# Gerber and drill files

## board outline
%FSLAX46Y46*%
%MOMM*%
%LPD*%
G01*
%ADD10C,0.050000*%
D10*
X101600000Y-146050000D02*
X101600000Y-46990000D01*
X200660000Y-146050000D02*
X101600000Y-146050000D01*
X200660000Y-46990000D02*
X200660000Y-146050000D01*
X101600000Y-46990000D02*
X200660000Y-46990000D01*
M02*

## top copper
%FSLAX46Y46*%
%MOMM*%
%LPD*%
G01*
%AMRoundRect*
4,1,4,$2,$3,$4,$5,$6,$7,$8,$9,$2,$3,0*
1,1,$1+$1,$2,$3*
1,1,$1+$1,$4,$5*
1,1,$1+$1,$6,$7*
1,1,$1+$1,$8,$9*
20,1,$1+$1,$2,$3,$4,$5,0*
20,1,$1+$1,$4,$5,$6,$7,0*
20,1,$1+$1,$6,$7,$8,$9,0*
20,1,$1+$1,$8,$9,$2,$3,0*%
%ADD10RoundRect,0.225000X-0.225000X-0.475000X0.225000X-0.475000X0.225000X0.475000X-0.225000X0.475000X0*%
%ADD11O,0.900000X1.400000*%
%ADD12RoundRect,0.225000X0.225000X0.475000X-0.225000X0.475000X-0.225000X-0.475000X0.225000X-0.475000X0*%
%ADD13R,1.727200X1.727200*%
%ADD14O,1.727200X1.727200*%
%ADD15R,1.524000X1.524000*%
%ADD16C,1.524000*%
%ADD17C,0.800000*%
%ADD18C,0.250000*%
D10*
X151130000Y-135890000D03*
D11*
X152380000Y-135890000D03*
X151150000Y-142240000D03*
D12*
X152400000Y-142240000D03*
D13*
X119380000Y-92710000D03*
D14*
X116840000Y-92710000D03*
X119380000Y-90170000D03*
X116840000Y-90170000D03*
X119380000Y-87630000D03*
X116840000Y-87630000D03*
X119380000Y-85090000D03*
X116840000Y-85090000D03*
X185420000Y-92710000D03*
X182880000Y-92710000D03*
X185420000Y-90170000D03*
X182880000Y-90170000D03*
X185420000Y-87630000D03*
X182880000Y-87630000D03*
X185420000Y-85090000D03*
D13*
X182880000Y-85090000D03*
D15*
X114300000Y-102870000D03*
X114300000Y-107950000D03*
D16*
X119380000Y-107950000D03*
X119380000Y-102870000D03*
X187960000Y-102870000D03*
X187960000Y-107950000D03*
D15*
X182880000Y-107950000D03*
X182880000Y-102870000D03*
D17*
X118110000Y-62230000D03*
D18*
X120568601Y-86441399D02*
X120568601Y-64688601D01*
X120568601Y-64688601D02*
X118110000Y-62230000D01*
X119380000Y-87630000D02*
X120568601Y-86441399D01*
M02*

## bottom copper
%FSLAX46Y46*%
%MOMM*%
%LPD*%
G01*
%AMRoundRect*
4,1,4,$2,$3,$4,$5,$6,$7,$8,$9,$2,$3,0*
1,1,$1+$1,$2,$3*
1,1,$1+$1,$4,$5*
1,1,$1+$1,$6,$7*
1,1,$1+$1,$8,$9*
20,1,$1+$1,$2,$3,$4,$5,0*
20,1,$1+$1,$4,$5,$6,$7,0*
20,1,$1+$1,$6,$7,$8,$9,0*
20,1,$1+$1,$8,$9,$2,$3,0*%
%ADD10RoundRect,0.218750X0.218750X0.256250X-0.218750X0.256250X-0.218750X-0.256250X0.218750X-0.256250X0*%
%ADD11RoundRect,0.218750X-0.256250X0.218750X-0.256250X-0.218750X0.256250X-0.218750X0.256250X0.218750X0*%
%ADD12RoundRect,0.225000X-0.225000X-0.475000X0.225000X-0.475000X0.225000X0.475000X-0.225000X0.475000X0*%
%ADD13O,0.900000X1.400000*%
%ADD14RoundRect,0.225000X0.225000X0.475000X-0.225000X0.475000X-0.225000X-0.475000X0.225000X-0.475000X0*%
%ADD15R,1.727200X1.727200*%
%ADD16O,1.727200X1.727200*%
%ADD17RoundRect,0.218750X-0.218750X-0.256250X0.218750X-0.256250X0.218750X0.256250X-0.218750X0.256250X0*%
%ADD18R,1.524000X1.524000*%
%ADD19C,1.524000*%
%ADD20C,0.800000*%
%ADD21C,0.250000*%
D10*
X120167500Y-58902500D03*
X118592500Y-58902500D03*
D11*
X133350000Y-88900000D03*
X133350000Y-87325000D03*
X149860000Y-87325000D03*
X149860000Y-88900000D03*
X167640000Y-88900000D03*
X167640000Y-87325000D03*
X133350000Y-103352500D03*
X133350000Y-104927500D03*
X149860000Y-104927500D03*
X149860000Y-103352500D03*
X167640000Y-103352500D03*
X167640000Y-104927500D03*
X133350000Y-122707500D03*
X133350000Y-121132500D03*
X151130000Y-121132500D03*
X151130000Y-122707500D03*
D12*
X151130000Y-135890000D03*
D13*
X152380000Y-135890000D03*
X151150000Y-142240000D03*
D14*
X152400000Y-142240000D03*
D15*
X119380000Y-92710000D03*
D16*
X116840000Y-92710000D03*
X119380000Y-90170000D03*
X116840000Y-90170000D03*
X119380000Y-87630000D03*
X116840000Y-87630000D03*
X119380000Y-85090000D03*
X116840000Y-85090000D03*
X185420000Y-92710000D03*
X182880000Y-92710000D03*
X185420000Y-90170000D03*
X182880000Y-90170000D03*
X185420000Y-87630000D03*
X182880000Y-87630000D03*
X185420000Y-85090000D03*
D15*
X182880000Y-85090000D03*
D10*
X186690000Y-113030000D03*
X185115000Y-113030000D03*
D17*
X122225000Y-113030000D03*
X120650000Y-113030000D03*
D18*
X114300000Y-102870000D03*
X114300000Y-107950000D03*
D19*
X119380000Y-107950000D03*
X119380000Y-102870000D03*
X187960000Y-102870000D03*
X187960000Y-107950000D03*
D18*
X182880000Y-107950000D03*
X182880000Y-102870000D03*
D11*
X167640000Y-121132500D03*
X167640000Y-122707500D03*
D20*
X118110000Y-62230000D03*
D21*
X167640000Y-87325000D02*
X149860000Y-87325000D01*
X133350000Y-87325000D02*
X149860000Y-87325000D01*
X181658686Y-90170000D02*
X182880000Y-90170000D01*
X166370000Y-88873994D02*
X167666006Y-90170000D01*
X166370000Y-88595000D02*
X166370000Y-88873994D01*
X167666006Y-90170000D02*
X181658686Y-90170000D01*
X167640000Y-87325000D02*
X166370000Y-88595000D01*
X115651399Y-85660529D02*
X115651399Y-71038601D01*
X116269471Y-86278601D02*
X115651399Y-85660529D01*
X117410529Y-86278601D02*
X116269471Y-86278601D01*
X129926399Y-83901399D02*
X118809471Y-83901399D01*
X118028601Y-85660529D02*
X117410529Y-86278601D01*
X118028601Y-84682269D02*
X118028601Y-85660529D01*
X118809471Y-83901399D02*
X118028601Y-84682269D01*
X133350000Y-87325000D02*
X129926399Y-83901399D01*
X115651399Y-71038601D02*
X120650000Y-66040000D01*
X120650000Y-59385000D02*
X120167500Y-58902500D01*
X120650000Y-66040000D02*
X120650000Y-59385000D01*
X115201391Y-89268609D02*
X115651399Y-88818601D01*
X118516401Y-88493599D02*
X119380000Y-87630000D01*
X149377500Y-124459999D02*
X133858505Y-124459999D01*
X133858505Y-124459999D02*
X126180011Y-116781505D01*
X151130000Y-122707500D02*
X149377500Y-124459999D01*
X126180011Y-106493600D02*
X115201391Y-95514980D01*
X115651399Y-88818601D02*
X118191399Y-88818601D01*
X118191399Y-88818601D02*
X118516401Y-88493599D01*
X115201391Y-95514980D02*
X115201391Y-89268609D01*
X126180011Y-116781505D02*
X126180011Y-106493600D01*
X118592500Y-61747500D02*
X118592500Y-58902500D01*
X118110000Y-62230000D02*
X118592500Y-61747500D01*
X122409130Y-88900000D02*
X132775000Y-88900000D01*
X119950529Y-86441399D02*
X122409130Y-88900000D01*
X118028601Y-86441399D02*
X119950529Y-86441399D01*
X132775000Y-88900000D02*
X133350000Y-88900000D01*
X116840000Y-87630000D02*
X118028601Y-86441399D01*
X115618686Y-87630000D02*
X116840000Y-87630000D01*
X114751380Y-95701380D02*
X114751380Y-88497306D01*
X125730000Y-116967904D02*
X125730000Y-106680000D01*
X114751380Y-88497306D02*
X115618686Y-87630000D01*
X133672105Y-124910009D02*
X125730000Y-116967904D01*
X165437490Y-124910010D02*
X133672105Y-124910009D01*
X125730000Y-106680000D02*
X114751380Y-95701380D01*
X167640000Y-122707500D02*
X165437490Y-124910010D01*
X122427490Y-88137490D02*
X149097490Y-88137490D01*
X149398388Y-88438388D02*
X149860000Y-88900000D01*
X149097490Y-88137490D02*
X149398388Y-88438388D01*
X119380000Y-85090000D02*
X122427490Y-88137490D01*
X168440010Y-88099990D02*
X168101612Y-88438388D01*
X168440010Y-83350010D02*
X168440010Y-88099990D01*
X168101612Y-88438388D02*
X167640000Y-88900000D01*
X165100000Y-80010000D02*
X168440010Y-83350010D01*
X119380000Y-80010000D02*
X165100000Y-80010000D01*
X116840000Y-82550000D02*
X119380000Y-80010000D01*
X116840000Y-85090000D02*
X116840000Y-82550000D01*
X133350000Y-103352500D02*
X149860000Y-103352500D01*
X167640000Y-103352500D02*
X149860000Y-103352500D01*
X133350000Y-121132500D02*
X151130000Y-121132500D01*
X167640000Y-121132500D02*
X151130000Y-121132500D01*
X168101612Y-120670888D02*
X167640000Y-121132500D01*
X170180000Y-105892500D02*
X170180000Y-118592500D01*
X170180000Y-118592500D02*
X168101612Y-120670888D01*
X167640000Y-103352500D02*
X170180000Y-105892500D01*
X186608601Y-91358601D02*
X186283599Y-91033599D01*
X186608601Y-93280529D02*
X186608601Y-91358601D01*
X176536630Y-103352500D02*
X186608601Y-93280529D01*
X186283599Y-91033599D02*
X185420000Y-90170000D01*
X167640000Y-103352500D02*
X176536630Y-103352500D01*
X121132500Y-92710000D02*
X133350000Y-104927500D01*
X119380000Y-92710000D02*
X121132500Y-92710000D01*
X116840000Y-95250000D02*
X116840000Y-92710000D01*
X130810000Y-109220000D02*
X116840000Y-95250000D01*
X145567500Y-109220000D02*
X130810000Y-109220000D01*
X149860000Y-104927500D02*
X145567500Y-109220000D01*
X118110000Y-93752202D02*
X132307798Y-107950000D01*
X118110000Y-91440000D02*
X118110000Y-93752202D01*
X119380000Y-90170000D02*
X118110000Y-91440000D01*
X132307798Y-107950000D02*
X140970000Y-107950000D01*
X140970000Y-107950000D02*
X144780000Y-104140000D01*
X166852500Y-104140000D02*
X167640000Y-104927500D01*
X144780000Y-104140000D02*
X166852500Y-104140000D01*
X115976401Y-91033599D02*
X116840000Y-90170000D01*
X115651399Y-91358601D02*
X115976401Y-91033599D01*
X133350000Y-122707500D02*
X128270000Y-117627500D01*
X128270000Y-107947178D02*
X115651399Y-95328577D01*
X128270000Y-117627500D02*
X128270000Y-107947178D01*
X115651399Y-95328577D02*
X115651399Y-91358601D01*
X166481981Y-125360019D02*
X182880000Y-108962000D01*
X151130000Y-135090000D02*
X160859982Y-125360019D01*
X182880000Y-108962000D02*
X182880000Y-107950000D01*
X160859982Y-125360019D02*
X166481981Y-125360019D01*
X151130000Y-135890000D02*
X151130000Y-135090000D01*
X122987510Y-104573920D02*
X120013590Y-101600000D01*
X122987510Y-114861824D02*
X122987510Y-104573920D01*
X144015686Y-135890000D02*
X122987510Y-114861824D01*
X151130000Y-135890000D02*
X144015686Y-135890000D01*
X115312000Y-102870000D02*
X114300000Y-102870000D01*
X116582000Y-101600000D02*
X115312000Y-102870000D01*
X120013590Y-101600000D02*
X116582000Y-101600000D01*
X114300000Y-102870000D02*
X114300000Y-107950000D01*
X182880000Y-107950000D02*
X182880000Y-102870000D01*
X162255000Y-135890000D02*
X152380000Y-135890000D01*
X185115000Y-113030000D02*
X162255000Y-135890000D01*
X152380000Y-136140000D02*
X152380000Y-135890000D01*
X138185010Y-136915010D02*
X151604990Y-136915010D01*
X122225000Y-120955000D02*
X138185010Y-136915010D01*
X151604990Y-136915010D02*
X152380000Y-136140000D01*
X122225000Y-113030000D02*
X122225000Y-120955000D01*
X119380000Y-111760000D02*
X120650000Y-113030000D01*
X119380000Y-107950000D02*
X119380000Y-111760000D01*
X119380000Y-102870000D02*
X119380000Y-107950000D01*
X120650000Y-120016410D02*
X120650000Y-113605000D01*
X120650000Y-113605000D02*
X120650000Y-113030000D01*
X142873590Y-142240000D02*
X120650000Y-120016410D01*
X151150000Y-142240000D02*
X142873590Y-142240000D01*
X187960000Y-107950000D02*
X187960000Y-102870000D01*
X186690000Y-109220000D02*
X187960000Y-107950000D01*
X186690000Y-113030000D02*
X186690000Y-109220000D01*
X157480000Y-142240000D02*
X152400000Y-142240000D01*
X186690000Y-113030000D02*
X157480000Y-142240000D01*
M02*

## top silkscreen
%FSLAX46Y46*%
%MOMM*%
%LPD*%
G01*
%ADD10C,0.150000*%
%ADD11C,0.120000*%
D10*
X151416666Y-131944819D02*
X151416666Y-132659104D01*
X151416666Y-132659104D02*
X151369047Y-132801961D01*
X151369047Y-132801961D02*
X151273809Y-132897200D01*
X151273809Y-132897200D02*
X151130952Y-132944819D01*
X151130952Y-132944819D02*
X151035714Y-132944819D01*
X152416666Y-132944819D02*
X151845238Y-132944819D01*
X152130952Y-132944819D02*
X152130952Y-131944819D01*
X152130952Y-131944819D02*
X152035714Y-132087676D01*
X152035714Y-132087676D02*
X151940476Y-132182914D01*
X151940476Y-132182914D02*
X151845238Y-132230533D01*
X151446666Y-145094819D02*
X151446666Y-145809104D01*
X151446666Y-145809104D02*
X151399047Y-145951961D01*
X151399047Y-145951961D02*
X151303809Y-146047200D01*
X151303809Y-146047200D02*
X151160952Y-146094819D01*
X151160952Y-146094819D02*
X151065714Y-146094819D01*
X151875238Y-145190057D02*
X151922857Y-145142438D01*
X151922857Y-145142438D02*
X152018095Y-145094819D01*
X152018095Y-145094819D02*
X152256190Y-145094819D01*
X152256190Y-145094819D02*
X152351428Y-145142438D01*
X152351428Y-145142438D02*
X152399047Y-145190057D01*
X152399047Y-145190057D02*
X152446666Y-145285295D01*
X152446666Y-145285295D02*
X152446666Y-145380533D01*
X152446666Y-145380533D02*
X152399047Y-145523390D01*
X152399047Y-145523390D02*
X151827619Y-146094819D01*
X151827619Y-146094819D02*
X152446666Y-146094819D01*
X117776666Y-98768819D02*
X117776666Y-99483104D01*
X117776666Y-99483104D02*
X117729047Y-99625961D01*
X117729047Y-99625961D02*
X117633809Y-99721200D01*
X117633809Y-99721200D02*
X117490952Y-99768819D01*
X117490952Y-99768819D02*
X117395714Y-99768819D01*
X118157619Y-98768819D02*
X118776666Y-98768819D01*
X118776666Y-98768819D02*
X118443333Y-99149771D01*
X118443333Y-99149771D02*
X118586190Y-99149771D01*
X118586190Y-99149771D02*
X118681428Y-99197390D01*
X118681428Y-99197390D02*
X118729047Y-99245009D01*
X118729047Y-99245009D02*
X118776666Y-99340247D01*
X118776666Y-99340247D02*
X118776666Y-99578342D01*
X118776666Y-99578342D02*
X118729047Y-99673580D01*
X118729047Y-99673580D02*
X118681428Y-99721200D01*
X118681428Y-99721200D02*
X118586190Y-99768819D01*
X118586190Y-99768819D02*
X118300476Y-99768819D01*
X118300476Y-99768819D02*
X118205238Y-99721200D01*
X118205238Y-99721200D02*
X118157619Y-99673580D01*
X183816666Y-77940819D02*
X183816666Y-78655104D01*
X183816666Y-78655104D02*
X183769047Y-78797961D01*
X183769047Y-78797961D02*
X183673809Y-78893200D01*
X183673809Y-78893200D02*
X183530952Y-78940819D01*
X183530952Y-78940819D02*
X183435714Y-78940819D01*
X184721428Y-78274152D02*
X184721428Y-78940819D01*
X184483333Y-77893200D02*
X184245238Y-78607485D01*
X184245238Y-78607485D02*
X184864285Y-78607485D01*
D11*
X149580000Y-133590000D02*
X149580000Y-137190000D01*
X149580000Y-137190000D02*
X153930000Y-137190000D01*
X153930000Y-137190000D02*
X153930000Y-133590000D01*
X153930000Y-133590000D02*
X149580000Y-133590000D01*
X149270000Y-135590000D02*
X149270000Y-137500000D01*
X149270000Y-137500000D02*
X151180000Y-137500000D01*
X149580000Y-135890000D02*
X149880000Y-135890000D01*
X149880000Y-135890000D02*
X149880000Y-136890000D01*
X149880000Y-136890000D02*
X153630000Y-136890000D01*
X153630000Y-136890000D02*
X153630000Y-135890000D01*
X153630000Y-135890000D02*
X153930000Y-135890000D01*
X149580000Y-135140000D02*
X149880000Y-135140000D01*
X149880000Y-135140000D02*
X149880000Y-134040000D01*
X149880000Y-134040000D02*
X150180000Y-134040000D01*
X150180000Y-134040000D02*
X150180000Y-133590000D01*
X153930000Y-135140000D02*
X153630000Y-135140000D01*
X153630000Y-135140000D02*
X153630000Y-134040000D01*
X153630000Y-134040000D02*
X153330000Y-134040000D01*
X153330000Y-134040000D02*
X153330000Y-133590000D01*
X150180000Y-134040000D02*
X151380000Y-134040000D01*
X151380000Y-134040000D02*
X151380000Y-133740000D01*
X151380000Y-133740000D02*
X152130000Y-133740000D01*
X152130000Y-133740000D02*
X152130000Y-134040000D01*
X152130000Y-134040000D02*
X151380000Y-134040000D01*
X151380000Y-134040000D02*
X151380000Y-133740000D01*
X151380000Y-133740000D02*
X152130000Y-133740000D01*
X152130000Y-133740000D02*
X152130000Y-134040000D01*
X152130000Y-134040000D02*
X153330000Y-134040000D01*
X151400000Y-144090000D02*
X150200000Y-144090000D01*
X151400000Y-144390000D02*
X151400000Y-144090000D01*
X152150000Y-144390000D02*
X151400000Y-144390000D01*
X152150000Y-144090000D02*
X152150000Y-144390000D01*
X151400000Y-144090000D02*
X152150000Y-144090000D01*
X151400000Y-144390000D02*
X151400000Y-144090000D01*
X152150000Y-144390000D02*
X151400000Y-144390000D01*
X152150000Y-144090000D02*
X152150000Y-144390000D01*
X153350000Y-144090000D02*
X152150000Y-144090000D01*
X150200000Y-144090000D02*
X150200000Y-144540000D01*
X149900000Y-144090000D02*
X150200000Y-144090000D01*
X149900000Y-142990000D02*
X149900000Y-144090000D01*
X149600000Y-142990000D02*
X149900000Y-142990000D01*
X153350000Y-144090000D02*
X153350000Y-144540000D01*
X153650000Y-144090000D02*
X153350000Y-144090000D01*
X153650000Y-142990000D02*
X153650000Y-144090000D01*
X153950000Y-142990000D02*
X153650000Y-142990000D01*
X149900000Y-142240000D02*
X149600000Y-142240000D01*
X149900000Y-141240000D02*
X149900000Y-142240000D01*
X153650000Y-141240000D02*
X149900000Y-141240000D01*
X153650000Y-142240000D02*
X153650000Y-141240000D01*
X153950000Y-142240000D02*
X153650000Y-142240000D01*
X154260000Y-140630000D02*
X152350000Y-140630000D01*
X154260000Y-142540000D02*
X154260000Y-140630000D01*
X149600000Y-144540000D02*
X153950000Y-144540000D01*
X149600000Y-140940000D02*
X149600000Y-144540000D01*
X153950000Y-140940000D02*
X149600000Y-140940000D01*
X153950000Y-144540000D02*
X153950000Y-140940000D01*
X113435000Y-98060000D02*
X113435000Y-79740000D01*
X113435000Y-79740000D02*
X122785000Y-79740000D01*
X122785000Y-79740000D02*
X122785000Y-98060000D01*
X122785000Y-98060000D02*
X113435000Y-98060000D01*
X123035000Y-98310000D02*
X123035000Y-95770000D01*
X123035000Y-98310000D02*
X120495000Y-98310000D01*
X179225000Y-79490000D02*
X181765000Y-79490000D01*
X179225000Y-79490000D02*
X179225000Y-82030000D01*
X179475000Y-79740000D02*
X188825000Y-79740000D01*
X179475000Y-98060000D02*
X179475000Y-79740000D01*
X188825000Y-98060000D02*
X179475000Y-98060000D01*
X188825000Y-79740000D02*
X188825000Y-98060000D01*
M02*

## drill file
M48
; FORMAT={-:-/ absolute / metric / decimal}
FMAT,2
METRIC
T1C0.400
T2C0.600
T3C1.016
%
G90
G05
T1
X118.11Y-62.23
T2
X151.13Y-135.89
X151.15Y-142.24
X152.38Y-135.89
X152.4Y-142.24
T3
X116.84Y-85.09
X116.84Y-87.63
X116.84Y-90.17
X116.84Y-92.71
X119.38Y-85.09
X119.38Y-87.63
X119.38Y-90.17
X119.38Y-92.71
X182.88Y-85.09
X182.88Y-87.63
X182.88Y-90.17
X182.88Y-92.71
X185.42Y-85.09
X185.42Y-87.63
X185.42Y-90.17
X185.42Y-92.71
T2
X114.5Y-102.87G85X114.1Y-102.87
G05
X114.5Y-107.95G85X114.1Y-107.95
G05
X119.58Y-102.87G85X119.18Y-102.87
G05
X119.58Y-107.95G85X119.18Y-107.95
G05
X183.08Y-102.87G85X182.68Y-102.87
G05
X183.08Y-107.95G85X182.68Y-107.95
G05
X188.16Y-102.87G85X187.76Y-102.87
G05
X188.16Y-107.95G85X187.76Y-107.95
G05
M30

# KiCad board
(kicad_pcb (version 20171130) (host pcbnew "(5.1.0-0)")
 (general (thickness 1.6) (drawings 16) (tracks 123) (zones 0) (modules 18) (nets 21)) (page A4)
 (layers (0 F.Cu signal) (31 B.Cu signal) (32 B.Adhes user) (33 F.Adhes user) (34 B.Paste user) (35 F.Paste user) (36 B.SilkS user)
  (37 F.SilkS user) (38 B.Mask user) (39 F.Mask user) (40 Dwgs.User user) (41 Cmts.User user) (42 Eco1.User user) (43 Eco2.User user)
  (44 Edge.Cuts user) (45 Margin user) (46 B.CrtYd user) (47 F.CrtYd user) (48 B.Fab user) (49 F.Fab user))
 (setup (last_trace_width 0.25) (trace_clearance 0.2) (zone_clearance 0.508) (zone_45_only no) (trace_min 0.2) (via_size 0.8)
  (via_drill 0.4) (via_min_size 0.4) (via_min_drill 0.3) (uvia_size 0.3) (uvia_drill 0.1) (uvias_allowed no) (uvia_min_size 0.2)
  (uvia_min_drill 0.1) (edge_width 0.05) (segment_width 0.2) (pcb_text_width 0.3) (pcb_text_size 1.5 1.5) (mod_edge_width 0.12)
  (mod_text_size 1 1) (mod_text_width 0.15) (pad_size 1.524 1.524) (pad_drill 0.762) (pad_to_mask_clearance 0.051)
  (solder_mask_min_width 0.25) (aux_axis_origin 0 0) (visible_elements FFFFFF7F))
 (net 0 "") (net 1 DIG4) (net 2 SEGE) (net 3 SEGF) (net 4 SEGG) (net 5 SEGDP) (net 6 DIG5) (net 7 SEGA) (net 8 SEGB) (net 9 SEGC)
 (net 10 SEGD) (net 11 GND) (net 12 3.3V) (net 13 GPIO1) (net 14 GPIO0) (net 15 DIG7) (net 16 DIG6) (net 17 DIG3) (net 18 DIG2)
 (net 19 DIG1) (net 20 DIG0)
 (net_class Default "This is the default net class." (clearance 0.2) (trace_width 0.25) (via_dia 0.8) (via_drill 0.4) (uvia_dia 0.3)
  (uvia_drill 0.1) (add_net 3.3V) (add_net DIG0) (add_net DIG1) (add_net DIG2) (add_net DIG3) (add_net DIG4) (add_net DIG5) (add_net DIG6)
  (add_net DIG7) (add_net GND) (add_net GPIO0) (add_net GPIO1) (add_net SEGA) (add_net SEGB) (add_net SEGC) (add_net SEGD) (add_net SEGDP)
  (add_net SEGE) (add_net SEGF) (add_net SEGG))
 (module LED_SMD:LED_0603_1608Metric (layer B.Cu) (at 119.38 58.9025 180)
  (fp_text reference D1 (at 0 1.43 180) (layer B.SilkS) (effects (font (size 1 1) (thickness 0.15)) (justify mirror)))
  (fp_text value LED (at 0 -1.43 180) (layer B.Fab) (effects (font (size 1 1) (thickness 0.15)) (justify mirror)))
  (pad 1 smd roundrect (at -0.7875 0 180) (size 0.875 0.95) (layers B.Cu B.Paste B.Mask) (roundrect_rratio 0.25) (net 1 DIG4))
  (pad 2 smd roundrect (at 0.7875 0 180) (size 0.875 0.95) (layers B.Cu B.Paste B.Mask) (roundrect_rratio 0.25) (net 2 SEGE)))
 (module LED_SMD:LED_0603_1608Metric (layer B.Cu) (at 133.35 88.1125 270)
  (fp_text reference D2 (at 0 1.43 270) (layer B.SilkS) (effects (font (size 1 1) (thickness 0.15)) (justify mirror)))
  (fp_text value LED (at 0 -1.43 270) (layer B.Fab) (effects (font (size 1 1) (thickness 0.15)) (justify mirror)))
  (pad 2 smd roundrect (at 0.7875 0 270) (size 0.875 0.95) (layers B.Cu B.Paste B.Mask) (roundrect_rratio 0.25) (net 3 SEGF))
  (pad 1 smd roundrect (at -0.7875 0 270) (size 0.875 0.95) (layers B.Cu B.Paste B.Mask) (roundrect_rratio 0.25) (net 1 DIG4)))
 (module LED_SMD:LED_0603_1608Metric (layer B.Cu) (at 149.86 88.1125 270)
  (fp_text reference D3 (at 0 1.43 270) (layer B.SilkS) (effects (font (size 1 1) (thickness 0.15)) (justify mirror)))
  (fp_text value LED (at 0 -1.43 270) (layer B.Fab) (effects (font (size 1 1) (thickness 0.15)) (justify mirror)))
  (pad 1 smd roundrect (at -0.7875 0 270) (size 0.875 0.95) (layers B.Cu B.Paste B.Mask) (roundrect_rratio 0.25) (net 1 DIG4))
  (pad 2 smd roundrect (at 0.7875 0 270) (size 0.875 0.95) (layers B.Cu B.Paste B.Mask) (roundrect_rratio 0.25) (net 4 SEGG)))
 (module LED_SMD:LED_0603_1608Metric (layer B.Cu) (at 167.64 88.1125 270)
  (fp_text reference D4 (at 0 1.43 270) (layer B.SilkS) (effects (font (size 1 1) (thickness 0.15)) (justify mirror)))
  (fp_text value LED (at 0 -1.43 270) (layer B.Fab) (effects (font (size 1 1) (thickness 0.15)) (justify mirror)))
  (pad 2 smd roundrect (at 0.7875 0 270) (size 0.875 0.95) (layers B.Cu B.Paste B.Mask) (roundrect_rratio 0.25) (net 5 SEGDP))
  (pad 1 smd roundrect (at -0.7875 0 270) (size 0.875 0.95) (layers B.Cu B.Paste B.Mask) (roundrect_rratio 0.25) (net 1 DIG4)))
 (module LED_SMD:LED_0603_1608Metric (layer B.Cu) (at 133.35 104.14 270)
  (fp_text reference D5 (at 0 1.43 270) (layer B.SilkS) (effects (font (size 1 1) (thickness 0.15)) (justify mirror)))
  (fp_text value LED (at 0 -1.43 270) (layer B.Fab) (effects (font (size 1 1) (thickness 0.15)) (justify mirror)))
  (pad 1 smd roundrect (at -0.7875 0 270) (size 0.875 0.95) (layers B.Cu B.Paste B.Mask) (roundrect_rratio 0.25) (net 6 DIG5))
  (pad 2 smd roundrect (at 0.7875 0 270) (size 0.875 0.95) (layers B.Cu B.Paste B.Mask) (roundrect_rratio 0.25) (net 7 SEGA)))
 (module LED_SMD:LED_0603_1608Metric (layer B.Cu) (at 149.86 104.14 270)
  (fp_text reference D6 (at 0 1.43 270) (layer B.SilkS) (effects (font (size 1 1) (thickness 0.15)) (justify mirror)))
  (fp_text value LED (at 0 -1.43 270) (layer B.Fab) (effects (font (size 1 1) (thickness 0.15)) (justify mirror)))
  (pad 2 smd roundrect (at 0.7875 0 270) (size 0.875 0.95) (layers B.Cu B.Paste B.Mask) (roundrect_rratio 0.25) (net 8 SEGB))
  (pad 1 smd roundrect (at -0.7875 0 270) (size 0.875 0.95) (layers B.Cu B.Paste B.Mask) (roundrect_rratio 0.25) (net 6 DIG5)))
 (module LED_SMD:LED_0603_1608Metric (layer B.Cu) (at 167.64 104.14 270)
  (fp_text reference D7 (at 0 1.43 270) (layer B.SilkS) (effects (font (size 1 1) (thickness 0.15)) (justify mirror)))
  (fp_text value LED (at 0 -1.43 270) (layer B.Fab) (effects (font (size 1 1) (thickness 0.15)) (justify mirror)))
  (pad 1 smd roundrect (at -0.7875 0 270) (size 0.875 0.95) (layers B.Cu B.Paste B.Mask) (roundrect_rratio 0.25) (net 6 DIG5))
  (pad 2 smd roundrect (at 0.7875 0 270) (size 0.875 0.95) (layers B.Cu B.Paste B.Mask) (roundrect_rratio 0.25) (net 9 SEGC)))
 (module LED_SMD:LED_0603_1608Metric (layer B.Cu) (at 133.35 121.92 270)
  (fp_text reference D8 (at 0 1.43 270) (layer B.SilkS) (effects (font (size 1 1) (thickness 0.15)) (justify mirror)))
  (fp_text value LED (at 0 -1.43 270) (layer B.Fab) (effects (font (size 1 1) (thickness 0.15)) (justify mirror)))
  (pad 2 smd roundrect (at 0.7875 0 270) (size 0.875 0.95) (layers B.Cu B.Paste B.Mask) (roundrect_rratio 0.25) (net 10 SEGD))
  (pad 1 smd roundrect (at -0.7875 0 270) (size 0.875 0.95) (layers B.Cu B.Paste B.Mask) (roundrect_rratio 0.25) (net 6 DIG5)))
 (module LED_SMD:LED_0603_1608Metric (layer B.Cu) (at 151.13 121.92 270)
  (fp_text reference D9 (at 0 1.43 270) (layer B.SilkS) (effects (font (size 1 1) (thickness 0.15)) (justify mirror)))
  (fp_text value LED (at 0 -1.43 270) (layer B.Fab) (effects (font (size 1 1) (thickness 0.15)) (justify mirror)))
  (pad 1 smd roundrect (at -0.7875 0 270) (size 0.875 0.95) (layers B.Cu B.Paste B.Mask) (roundrect_rratio 0.25) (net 6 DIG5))
  (pad 2 smd roundrect (at 0.7875 0 270) (size 0.875 0.95) (layers B.Cu B.Paste B.Mask) (roundrect_rratio 0.25) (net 2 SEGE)))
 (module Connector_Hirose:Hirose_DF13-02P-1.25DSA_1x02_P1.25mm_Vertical (layer F.Cu) (at 151.13 135.89)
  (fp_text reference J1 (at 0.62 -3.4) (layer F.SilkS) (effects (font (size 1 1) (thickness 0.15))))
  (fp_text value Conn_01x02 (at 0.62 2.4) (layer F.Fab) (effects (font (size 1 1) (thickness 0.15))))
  (fp_line (start -1.55 -2.3) (end -1.55 1.3) (layer F.SilkS) (width 0.12))
  (fp_line (start -1.55 1.3) (end 2.8 1.3) (layer F.SilkS) (width 0.12))
  (fp_line (start 2.8 1.3) (end 2.8 -2.3) (layer F.SilkS) (width 0.12))
  (fp_line (start 2.8 -2.3) (end -1.55 -2.3) (layer F.SilkS) (width 0.12))
  (fp_line (start -1.86 -0.3) (end -1.86 1.61) (layer F.SilkS) (width 0.12))
  (fp_line (start -1.86 1.61) (end 0.05 1.61) (layer F.SilkS) (width 0.12))
  (fp_line (start -1.55 0) (end -1.25 0) (layer F.SilkS) (width 0.12))
  (fp_line (start -1.25 0) (end -1.25 1) (layer F.SilkS) (width 0.12))
  (fp_line (start -1.25 1) (end 2.5 1) (layer F.SilkS) (width 0.12))
  (fp_line (start 2.5 1) (end 2.5 0) (layer F.SilkS) (width 0.12))
  (fp_line (start 2.5 0) (end 2.8 0) (layer F.SilkS) (width 0.12))
  (fp_line (start -1.55 -0.75) (end -1.25 -0.75) (layer F.SilkS) (width 0.12))
  (fp_line (start -1.25 -0.75) (end -1.25 -1.85) (layer F.SilkS) (width 0.12))
  (fp_line (start -1.25 -1.85) (end -0.95 -1.85) (layer F.SilkS) (width 0.12))
  (fp_line (start -0.95 -1.85) (end -0.95 -2.3) (layer F.SilkS) (width 0.12))
  (fp_line (start 2.8 -0.75) (end 2.5 -0.75) (layer F.SilkS) (width 0.12))
  (fp_line (start 2.5 -0.75) (end 2.5 -1.85) (layer F.SilkS) (width 0.12))
  (fp_line (start 2.5 -1.85) (end 2.2 -1.85) (layer F.SilkS) (width 0.12))
  (fp_line (start 2.2 -1.85) (end 2.2 -2.3) (layer F.SilkS) (width 0.12))
  (fp_line (start -0.95 -1.85) (end 0.25 -1.85) (layer F.SilkS) (width 0.12))
  (fp_line (start 0.25 -1.85) (end 0.25 -2.15) (layer F.SilkS) (width 0.12))
  (fp_line (start 0.25 -2.15) (end 1 -2.15) (layer F.SilkS) (width 0.12))
  (fp_line (start 1 -2.15) (end 1 -1.85) (layer F.SilkS) (width 0.12))
  (fp_line (start 1 -1.85) (end 0.25 -1.85) (layer F.SilkS) (width 0.12))
  (fp_line (start 0.25 -1.85) (end 0.25 -2.15) (layer F.SilkS) (width 0.12))
  (fp_line (start 0.25 -2.15) (end 1 -2.15) (layer F.SilkS) (width 0.12))
  (fp_line (start 1 -2.15) (end 1 -1.85) (layer F.SilkS) (width 0.12))
  (fp_line (start 1 -1.85) (end 2.2 -1.85) (layer F.SilkS) (width 0.12))
  (pad 1 thru_hole roundrect (at 0 0) (size 0.9 1.4) (drill 0.6) (layers *.Cu *.Mask) (roundrect_rratio 0.25) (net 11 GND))
  (pad 2 thru_hole oval (at 1.25 0) (size 0.9 1.4) (drill 0.6) (layers *.Cu *.Mask) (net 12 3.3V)))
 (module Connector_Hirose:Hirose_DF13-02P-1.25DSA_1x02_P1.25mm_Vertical (layer F.Cu) (at 152.4 142.24 180)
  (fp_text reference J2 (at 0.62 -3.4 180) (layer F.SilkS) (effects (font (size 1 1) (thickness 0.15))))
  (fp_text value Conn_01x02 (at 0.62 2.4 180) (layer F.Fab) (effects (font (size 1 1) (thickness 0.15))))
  (fp_line (start 1 -1.85) (end 2.2 -1.85) (layer F.SilkS) (width 0.12))
  (fp_line (start 1 -2.15) (end 1 -1.85) (layer F.SilkS) (width 0.12))
  (fp_line (start 0.25 -2.15) (end 1 -2.15) (layer F.SilkS) (width 0.12))
  (fp_line (start 0.25 -1.85) (end 0.25 -2.15) (layer F.SilkS) (width 0.12))
  (fp_line (start 1 -1.85) (end 0.25 -1.85) (layer F.SilkS) (width 0.12))
  (fp_line (start 1 -2.15) (end 1 -1.85) (layer F.SilkS) (width 0.12))
  (fp_line (start 0.25 -2.15) (end 1 -2.15) (layer F.SilkS) (width 0.12))
  (fp_line (start 0.25 -1.85) (end 0.25 -2.15) (layer F.SilkS) (width 0.12))
  (fp_line (start -0.95 -1.85) (end 0.25 -1.85) (layer F.SilkS) (width 0.12))
  (fp_line (start 2.2 -1.85) (end 2.2 -2.3) (layer F.SilkS) (width 0.12))
  (fp_line (start 2.5 -1.85) (end 2.2 -1.85) (layer F.SilkS) (width 0.12))
  (fp_line (start 2.5 -0.75) (end 2.5 -1.85) (layer F.SilkS) (width 0.12))
  (fp_line (start 2.8 -0.75) (end 2.5 -0.75) (layer F.SilkS) (width 0.12))
  (fp_line (start -0.95 -1.85) (end -0.95 -2.3) (layer F.SilkS) (width 0.12))
  (fp_line (start -1.25 -1.85) (end -0.95 -1.85) (layer F.SilkS) (width 0.12))
  (fp_line (start -1.25 -0.75) (end -1.25 -1.85) (layer F.SilkS) (width 0.12))
  (fp_line (start -1.55 -0.75) (end -1.25 -0.75) (layer F.SilkS) (width 0.12))
  (fp_line (start 2.5 0) (end 2.8 0) (layer F.SilkS) (width 0.12))
  (fp_line (start 2.5 1) (end 2.5 0) (layer F.SilkS) (width 0.12))
  (fp_line (start -1.25 1) (end 2.5 1) (layer F.SilkS) (width 0.12))
  (fp_line (start -1.25 0) (end -1.25 1) (layer F.SilkS) (width 0.12))
  (fp_line (start -1.55 0) (end -1.25 0) (layer F.SilkS) (width 0.12))
  (fp_line (start -1.86 1.61) (end 0.05 1.61) (layer F.SilkS) (width 0.12))
  (fp_line (start -1.86 -0.3) (end -1.86 1.61) (layer F.SilkS) (width 0.12))
  (fp_line (start 2.8 -2.3) (end -1.55 -2.3) (layer F.SilkS) (width 0.12))
  (fp_line (start 2.8 1.3) (end 2.8 -2.3) (layer F.SilkS) (width 0.12))
  (fp_line (start -1.55 1.3) (end 2.8 1.3) (layer F.SilkS) (width 0.12))
  (fp_line (start -1.55 -2.3) (end -1.55 1.3) (layer F.SilkS) (width 0.12))
  (pad 2 thru_hole oval (at 1.25 0 180) (size 0.9 1.4) (drill 0.6) (layers *.Cu *.Mask) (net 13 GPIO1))
  (pad 1 thru_hole roundrect (at 0 0 180) (size 0.9 1.4) (drill 0.6) (layers *.Cu *.Mask) (roundrect_rratio 0.25) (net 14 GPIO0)))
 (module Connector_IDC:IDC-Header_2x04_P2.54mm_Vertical (layer F.Cu) (at 119.38 92.71 180)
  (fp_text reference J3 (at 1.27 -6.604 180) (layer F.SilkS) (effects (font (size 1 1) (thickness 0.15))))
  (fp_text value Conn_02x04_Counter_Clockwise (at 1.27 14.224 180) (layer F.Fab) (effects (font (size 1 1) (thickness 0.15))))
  (fp_line (start 5.945 -5.35) (end 5.945 12.97) (layer F.SilkS) (width 0.12))
  (fp_line (start 5.945 12.97) (end -3.405 12.97) (layer F.SilkS) (width 0.12))
  (fp_line (start -3.405 12.97) (end -3.405 -5.35) (layer F.SilkS) (width 0.12))
  (fp_line (start -3.405 -5.35) (end 5.945 -5.35) (layer F.SilkS) (width 0.12))
  (fp_line (start -3.655 -5.6) (end -3.655 -3.06) (layer F.SilkS) (width 0.12))
  (fp_line (start -3.655 -5.6) (end -1.115 -5.6) (layer F.SilkS) (width 0.12))
  (pad 1 thru_hole rect (at 0 0 180) (size 1.7272 1.7272) (drill 1.016) (layers *.Cu *.Mask) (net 7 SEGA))
  (pad 2 thru_hole oval (at 2.54 0 180) (size 1.7272 1.7272) (drill 1.016) (layers *.Cu *.Mask) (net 8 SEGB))
  (pad 3 thru_hole oval (at 0 2.54 180) (size 1.7272 1.7272) (drill 1.016) (layers *.Cu *.Mask) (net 9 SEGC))
  (pad 4 thru_hole oval (at 2.54 2.54 180) (size 1.7272 1.7272) (drill 1.016) (layers *.Cu *.Mask) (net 10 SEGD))
  (pad 5 thru_hole oval (at 0 5.08 180) (size 1.7272 1.7272) (drill 1.016) (layers *.Cu *.Mask) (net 2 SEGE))
  (pad 6 thru_hole oval (at 2.54 5.08 180) (size 1.7272 1.7272) (drill 1.016) (layers *.Cu *.Mask) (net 3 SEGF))
  (pad 7 thru_hole oval (at 0 7.62 180) (size 1.7272 1.7272) (drill 1.016) (layers *.Cu *.Mask) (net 4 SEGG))
  (pad 8 thru_hole oval (at 2.54 7.62 180) (size 1.7272 1.7272) (drill 1.016) (layers *.Cu *.Mask) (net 5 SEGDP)))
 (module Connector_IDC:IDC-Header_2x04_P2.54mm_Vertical (layer F.Cu) (at 182.88 85.09)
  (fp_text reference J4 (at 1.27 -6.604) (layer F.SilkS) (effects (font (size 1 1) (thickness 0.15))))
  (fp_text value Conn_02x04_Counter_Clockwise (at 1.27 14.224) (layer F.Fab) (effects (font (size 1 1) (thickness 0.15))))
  (fp_line (start -3.655 -5.6) (end -1.115 -5.6) (layer F.SilkS) (width 0.12))
  (fp_line (start -3.655 -5.6) (end -3.655 -3.06) (layer F.SilkS) (width 0.12))
  (fp_line (start -3.405 -5.35) (end 5.945 -5.35) (layer F.SilkS) (width 0.12))
  (fp_line (start -3.405 12.97) (end -3.405 -5.35) (layer F.SilkS) (width 0.12))
  (fp_line (start 5.945 12.97) (end -3.405 12.97) (layer F.SilkS) (width 0.12))
  (fp_line (start 5.945 -5.35) (end 5.945 12.97) (layer F.SilkS) (width 0.12))
  (pad 8 thru_hole oval (at 2.54 7.62) (size 1.7272 1.7272) (drill 1.016) (layers *.Cu *.Mask) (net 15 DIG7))
  (pad 7 thru_hole oval (at 0 7.62) (size 1.7272 1.7272) (drill 1.016) (layers *.Cu *.Mask) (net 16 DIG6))
  (pad 6 thru_hole oval (at 2.54 5.08) (size 1.7272 1.7272) (drill 1.016) (layers *.Cu *.Mask) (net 6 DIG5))
  (pad 5 thru_hole oval (at 0 5.08) (size 1.7272 1.7272) (drill 1.016) (layers *.Cu *.Mask) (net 1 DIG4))
  (pad 4 thru_hole oval (at 2.54 2.54) (size 1.7272 1.7272) (drill 1.016) (layers *.Cu *.Mask) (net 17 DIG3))
  (pad 3 thru_hole oval (at 0 2.54) (size 1.7272 1.7272) (drill 1.016) (layers *.Cu *.Mask) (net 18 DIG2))
  (pad 2 thru_hole oval (at 2.54 0) (size 1.7272 1.7272) (drill 1.016) (layers *.Cu *.Mask) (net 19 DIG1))
  (pad 1 thru_hole rect (at 0 0) (size 1.7272 1.7272) (drill 1.016) (layers *.Cu *.Mask) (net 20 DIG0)))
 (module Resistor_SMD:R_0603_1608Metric (layer B.Cu) (at 185.9025 113.03 180)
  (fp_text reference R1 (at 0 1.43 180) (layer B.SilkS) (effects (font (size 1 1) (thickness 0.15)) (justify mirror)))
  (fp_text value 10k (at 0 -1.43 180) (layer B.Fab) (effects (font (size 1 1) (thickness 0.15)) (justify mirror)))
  (pad 1 smd roundrect (at -0.7875 0 180) (size 0.875 0.95) (layers B.Cu B.Paste B.Mask) (roundrect_rratio 0.25) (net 14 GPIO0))
  (pad 2 smd roundrect (at 0.7875 0 180) (size 0.875 0.95) (layers B.Cu B.Paste B.Mask) (roundrect_rratio 0.25) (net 12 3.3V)))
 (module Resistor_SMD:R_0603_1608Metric (layer B.Cu) (at 121.4375 113.03)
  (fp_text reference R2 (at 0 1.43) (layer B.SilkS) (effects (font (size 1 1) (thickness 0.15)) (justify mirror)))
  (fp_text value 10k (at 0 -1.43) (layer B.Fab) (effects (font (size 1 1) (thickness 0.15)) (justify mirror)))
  (pad 2 smd roundrect (at 0.7875 0) (size 0.875 0.95) (layers B.Cu B.Paste B.Mask) (roundrect_rratio 0.25) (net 12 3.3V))
  (pad 1 smd roundrect (at -0.7875 0) (size 0.875 0.95) (layers B.Cu B.Paste B.Mask) (roundrect_rratio 0.25) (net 13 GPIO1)))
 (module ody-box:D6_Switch (layer B.Cu) (at 116.84 105.41 270)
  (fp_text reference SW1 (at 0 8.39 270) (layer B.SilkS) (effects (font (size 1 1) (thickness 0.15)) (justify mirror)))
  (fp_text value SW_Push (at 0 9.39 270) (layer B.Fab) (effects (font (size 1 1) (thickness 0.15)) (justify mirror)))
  (pad 1 thru_hole rect (at -2.54 2.54 270) (size 1.524 1.524) (drill oval 0.6 1) (layers *.Cu *.Mask) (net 11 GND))
  (pad 1 thru_hole rect (at 2.54 2.54 270) (size 1.524 1.524) (drill oval 0.6 1) (layers *.Cu *.Mask) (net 11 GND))
  (pad 2 thru_hole circle (at 2.54 -2.54 270) (size 1.524 1.524) (drill oval 0.6 1) (layers *.Cu *.Mask) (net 13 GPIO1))
  (pad 2 thru_hole circle (at -2.54 -2.54 270) (size 1.524 1.524) (drill oval 0.6 1) (layers *.Cu *.Mask) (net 13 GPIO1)))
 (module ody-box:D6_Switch (layer B.Cu) (at 185.42 105.41 270)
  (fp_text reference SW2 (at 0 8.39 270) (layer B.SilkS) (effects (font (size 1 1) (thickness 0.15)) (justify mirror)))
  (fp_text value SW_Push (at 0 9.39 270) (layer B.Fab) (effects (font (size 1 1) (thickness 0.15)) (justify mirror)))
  (pad 2 thru_hole circle (at -2.54 -2.54 270) (size 1.524 1.524) (drill oval 0.6 1) (layers *.Cu *.Mask) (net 14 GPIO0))
  (pad 2 thru_hole circle (at 2.54 -2.54 270) (size 1.524 1.524) (drill oval 0.6 1) (layers *.Cu *.Mask) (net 14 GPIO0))
  (pad 1 thru_hole rect (at 2.54 2.54 270) (size 1.524 1.524) (drill oval 0.6 1) (layers *.Cu *.Mask) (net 11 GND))
  (pad 1 thru_hole rect (at -2.54 2.54 270) (size 1.524 1.524) (drill oval 0.6 1) (layers *.Cu *.Mask) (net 11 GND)))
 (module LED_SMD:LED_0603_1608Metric (layer B.Cu) (at 167.64 121.92 270)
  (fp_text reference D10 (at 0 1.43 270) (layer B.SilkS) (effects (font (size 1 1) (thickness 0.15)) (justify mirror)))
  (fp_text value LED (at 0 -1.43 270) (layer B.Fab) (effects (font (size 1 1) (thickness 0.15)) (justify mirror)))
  (pad 1 smd roundrect (at -0.7875 0 270) (size 0.875 0.95) (layers B.Cu B.Paste B.Mask) (roundrect_rratio 0.25) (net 6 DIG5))
  (pad 2 smd roundrect (at 0.7875 0 270) (size 0.875 0.95) (layers B.Cu B.Paste B.Mask) (roundrect_rratio 0.25) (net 3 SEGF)))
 (gr_line (start 101.6 146.05) (end 101.6 46.99) (layer Edge.Cuts) (width 0.05))
 (gr_line (start 200.66 146.05) (end 101.6 146.05) (layer Edge.Cuts) (width 0.05))
 (gr_line (start 200.66 46.99) (end 200.66 146.05) (layer Edge.Cuts) (width 0.05))
 (gr_line (start 101.6 46.99) (end 200.66 46.99) (layer Edge.Cuts) (width 0.05))
 (segment (start 167.64 87.325) (end 149.86 87.325) (width 0.25) (layer B.Cu) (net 1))
 (segment (start 133.35 87.325) (end 149.86 87.325) (width 0.25) (layer B.Cu) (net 1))
 (segment (start 181.658686 90.17) (end 182.88 90.17) (width 0.25) (layer B.Cu) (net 1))
 (segment (start 166.37 88.873994) (end 167.666006 90.17) (width 0.25) (layer B.Cu) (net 1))
 (segment (start 166.37 88.595) (end 166.37 88.873994) (width 0.25) (layer B.Cu) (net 1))
 (segment (start 167.666006 90.17) (end 181.658686 90.17) (width 0.25) (layer B.Cu) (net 1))
 (segment (start 167.64 87.325) (end 166.37 88.595) (width 0.25) (layer B.Cu) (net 1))
 (segment (start 115.651399 85.660529) (end 115.651399 71.038601) (width 0.25) (layer B.Cu) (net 1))
 (segment (start 116.269471 86.278601) (end 115.651399 85.660529) (width 0.25) (layer B.Cu) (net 1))
 (segment (start 117.410529 86.278601) (end 116.269471 86.278601) (width 0.25) (layer B.Cu) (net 1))
 (segment (start 129.926399 83.901399) (end 118.809471 83.901399) (width 0.25) (layer B.Cu) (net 1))
 (segment (start 118.028601 85.660529) (end 117.410529 86.278601) (width 0.25) (layer B.Cu) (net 1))
 (segment (start 118.028601 84.682269) (end 118.028601 85.660529) (width 0.25) (layer B.Cu) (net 1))
 (segment (start 118.809471 83.901399) (end 118.028601 84.682269) (width 0.25) (layer B.Cu) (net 1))
 (segment (start 133.35 87.325) (end 129.926399 83.901399) (width 0.25) (layer B.Cu) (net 1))
 (segment (start 115.651399 71.038601) (end 120.65 66.04) (width 0.25) (layer B.Cu) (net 1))
 (segment (start 120.65 59.385) (end 120.1675 58.9025) (width 0.25) (layer B.Cu) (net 1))
 (segment (start 120.65 66.04) (end 120.65 59.385) (width 0.25) (layer B.Cu) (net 1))
 (segment (start 115.201391 89.268609) (end 115.651399 88.818601) (width 0.25) (layer B.Cu) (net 2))
 (segment (start 118.516401 88.493599) (end 119.38 87.63) (width 0.25) (layer B.Cu) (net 2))
 (segment (start 149.3775 124.459999) (end 133.858505 124.459999) (width 0.25) (layer B.Cu) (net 2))
 (segment (start 133.858505 124.459999) (end 126.180011 116.781505) (width 0.25) (layer B.Cu) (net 2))
 (segment (start 151.13 122.7075) (end 149.3775 124.459999) (width 0.25) (layer B.Cu) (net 2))
 (segment (start 126.180011 106.4936) (end 115.201391 95.51498) (width 0.25) (layer B.Cu) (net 2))
 (segment (start 115.651399 88.818601) (end 118.191399 88.818601) (width 0.25) (layer B.Cu) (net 2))
 (segment (start 118.191399 88.818601) (end 118.516401 88.493599) (width 0.25) (layer B.Cu) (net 2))
 (segment (start 115.201391 95.51498) (end 115.201391 89.268609) (width 0.25) (layer B.Cu) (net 2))
 (segment (start 126.180011 116.781505) (end 126.180011 106.4936) (width 0.25) (layer B.Cu) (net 2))
 (segment (start 120.568601 86.441399) (end 120.568601 64.688601) (width 0.25) (layer F.Cu) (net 2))
 (via (at 118.11 62.23) (size 0.8) (drill 0.4) (layers F.Cu B.Cu) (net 2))
 (segment (start 120.568601 64.688601) (end 118.11 62.23) (width 0.25) (layer F.Cu) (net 2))
 (segment (start 119.38 87.63) (end 120.568601 86.441399) (width 0.25) (layer F.Cu) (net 2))
 (segment (start 118.5925 61.7475) (end 118.5925 58.9025) (width 0.25) (layer B.Cu) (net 2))
 (segment (start 118.11 62.23) (end 118.5925 61.7475) (width 0.25) (layer B.Cu) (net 2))
 (segment (start 122.40913 88.9) (end 132.775 88.9) (width 0.25) (layer B.Cu) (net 3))
 (segment (start 119.950529 86.441399) (end 122.40913 88.9) (width 0.25) (layer B.Cu) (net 3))
 (segment (start 118.028601 86.441399) (end 119.950529 86.441399) (width 0.25) (layer B.Cu) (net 3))
 (segment (start 132.775 88.9) (end 133.35 88.9) (width 0.25) (layer B.Cu) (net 3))
 (segment (start 116.84 87.63) (end 118.028601 86.441399) (width 0.25) (layer B.Cu) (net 3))
 (segment (start 115.618686 87.63) (end 116.84 87.63) (width 0.25) (layer B.Cu) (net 3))
 (segment (start 114.75138 95.70138) (end 114.75138 88.497306) (width 0.25) (layer B.Cu) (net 3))
 (segment (start 125.73 116.967904) (end 125.73 106.68) (width 0.25) (layer B.Cu) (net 3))
 (segment (start 114.75138 88.497306) (end 115.618686 87.63) (width 0.25) (layer B.Cu) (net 3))
 (segment (start 133.672105 124.910009) (end 125.73 116.967904) (width 0.25) (layer B.Cu) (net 3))
 (segment (start 165.43749 124.91001) (end 133.672105 124.910009) (width 0.25) (layer B.Cu) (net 3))
 (segment (start 125.73 106.68) (end 114.75138 95.70138) (width 0.25) (layer B.Cu) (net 3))
 (segment (start 167.64 122.7075) (end 165.43749 124.91001) (width 0.25) (layer B.Cu) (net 3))
 (segment (start 122.42749 88.13749) (end 149.09749 88.13749) (width 0.25) (layer B.Cu) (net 4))
 (segment (start 149.398388 88.438388) (end 149.86 88.9) (width 0.25) (layer B.Cu) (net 4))
 (segment (start 149.09749 88.13749) (end 149.398388 88.438388) (width 0.25) (layer B.Cu) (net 4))
 (segment (start 119.38 85.09) (end 122.42749 88.13749) (width 0.25) (layer B.Cu) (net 4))
 (segment (start 168.44001 88.09999) (end 168.101612 88.438388) (width 0.25) (layer B.Cu) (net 5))
 (segment (start 168.44001 83.35001) (end 168.44001 88.09999) (width 0.25) (layer B.Cu) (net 5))
 (segment (start 168.101612 88.438388) (end 167.64 88.9) (width 0.25) (layer B.Cu) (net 5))
 (segment (start 165.1 80.01) (end 168.44001 83.35001) (width 0.25) (layer B.Cu) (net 5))
 (segment (start 119.38 80.01) (end 165.1 80.01) (width 0.25) (layer B.Cu) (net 5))
 (segment (start 116.84 82.55) (end 119.38 80.01) (width 0.25) (layer B.Cu) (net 5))
 (segment (start 116.84 85.09) (end 116.84 82.55) (width 0.25) (layer B.Cu) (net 5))
 (segment (start 133.35 103.3525) (end 149.86 103.3525) (width 0.25) (layer B.Cu) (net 6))
 (segment (start 167.64 103.3525) (end 149.86 103.3525) (width 0.25) (layer B.Cu) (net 6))
 (segment (start 133.35 121.1325) (end 151.13 121.1325) (width 0.25) (layer B.Cu) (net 6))
 (segment (start 167.64 121.1325) (end 151.13 121.1325) (width 0.25) (layer B.Cu) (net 6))
 (segment (start 168.101612 120.670888) (end 167.64 121.1325) (width 0.25) (layer B.Cu) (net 6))
 (segment (start 170.18 105.8925) (end 170.18 118.5925) (width 0.25) (layer B.Cu) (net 6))
 (segment (start 170.18 118.5925) (end 168.101612 120.670888) (width 0.25) (layer B.Cu) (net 6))
 (segment (start 167.64 103.3525) (end 170.18 105.8925) (width 0.25) (layer B.Cu) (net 6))
 (segment (start 186.608601 91.358601) (end 186.283599 91.033599) (width 0.25) (layer B.Cu) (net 6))
 (segment (start 186.608601 93.280529) (end 186.608601 91.358601) (width 0.25) (layer B.Cu) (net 6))
 (segment (start 176.53663 103.3525) (end 186.608601 93.280529) (width 0.25) (layer B.Cu) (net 6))
 (segment (start 186.283599 91.033599) (end 185.42 90.17) (width 0.25) (layer B.Cu) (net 6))
 (segment (start 167.64 103.3525) (end 176.53663 103.3525) (width 0.25) (layer B.Cu) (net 6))
 (segment (start 121.1325 92.71) (end 133.35 104.9275) (width 0.25) (layer B.Cu) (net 7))
 (segment (start 119.38 92.71) (end 121.1325 92.71) (width 0.25) (layer B.Cu) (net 7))
 (segment (start 116.84 95.25) (end 116.84 92.71) (width 0.25) (layer B.Cu) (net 8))
 (segment (start 130.81 109.22) (end 116.84 95.25) (width 0.25) (layer B.Cu) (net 8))
 (segment (start 145.5675 109.22) (end 130.81 109.22) (width 0.25) (layer B.Cu) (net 8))
 (segment (start 149.86 104.9275) (end 145.5675 109.22) (width 0.25) (layer B.Cu) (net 8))
 (segment (start 118.11 93.752202) (end 132.307798 107.95) (width 0.25) (layer B.Cu) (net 9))
 (segment (start 118.11 91.44) (end 118.11 93.752202) (width 0.25) (layer B.Cu) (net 9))
 (segment (start 119.38 90.17) (end 118.11 91.44) (width 0.25) (layer B.Cu) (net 9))
 (segment (start 132.307798 107.95) (end 140.97 107.95) (width 0.25) (layer B.Cu) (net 9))
 (segment (start 140.97 107.95) (end 144.78 104.14) (width 0.25) (layer B.Cu) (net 9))
 (segment (start 166.8525 104.14) (end 167.64 104.9275) (width 0.25) (layer B.Cu) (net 9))
 (segment (start 144.78 104.14) (end 166.8525 104.14) (width 0.25) (layer B.Cu) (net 9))
 (segment (start 115.976401 91.033599) (end 116.84 90.17) (width 0.25) (layer B.Cu) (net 10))
 (segment (start 115.651399 91.358601) (end 115.976401 91.033599) (width 0.25) (layer B.Cu) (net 10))
 (segment (start 133.35 122.7075) (end 128.27 117.6275) (width 0.25) (layer B.Cu) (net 10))
 (segment (start 128.27 107.947178) (end 115.651399 95.328577) (width 0.25) (layer B.Cu) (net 10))
 (segment (start 128.27 117.6275) (end 128.27 107.947178) (width 0.25) (layer B.Cu) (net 10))
 (segment (start 115.651399 95.328577) (end 115.651399 91.358601) (width 0.25) (layer B.Cu) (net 10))
 (segment (start 166.481981 125.360019) (end 182.88 108.962) (width 0.25) (layer B.Cu) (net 11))
 (segment (start 151.13 135.09) (end 160.859982 125.360019) (width 0.25) (layer B.Cu) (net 11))
 (segment (start 182.88 108.962) (end 182.88 107.95) (width 0.25) (layer B.Cu) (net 11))
 (segment (start 160.859982 125.360019) (end 166.481981 125.360019) (width 0.25) (layer B.Cu) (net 11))
 (segment (start 151.13 135.89) (end 151.13 135.09) (width 0.25) (layer B.Cu) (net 11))
 (segment (start 122.98751 104.57392) (end 120.01359 101.6) (width 0.25) (layer B.Cu) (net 11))
 (segment (start 122.98751 114.861824) (end 122.98751 104.57392) (width 0.25) (layer B.Cu) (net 11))
 (segment (start 144.015686 135.89) (end 122.98751 114.861824) (width 0.25) (layer B.Cu) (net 11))
 (segment (start 151.13 135.89) (end 144.015686 135.89) (width 0.25) (layer B.Cu) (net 11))
 (segment (start 115.312 102.87) (end 114.3 102.87) (width 0.25) (layer B.Cu) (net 11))
 (segment (start 116.582 101.6) (end 115.312 102.87) (width 0.25) (layer B.Cu) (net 11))
 (segment (start 120.01359 101.6) (end 116.582 101.6) (width 0.25) (layer B.Cu) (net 11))
 (segment (start 114.3 102.87) (end 114.3 107.95) (width 0.25) (layer B.Cu) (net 11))
 (segment (start 182.88 107.95) (end 182.88 102.87) (width 0.25) (layer B.Cu) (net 11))
 (segment (start 162.255 135.89) (end 152.38 135.89) (width 0.25) (layer B.Cu) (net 12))
 (segment (start 185.115 113.03) (end 162.255 135.89) (width 0.25) (layer B.Cu) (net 12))
 (segment (start 152.38 136.14) (end 152.38 135.89) (width 0.25) (layer B.Cu) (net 12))
 (segment (start 138.18501 136.91501) (end 151.60499 136.91501) (width 0.25) (layer B.Cu) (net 12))
 (segment (start 122.225 120.955) (end 138.18501 136.91501) (width 0.25) (layer B.Cu) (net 12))
 (segment (start 151.60499 136.91501) (end 152.38 136.14) (width 0.25) (layer B.Cu) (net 12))
 (segment (start 122.225 113.03) (end 122.225 120.955) (width 0.25) (layer B.Cu) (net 12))
 (segment (start 119.38 111.76) (end 120.65 113.03) (width 0.25) (layer B.Cu) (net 13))
 (segment (start 119.38 107.95) (end 119.38 111.76) (width 0.25) (layer B.Cu) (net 13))
 (segment (start 119.38 102.87) (end 119.38 107.95) (width 0.25) (layer B.Cu) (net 13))
 (segment (start 120.65 120.01641) (end 120.65 113.605) (width 0.25) (layer B.Cu) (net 13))
 (segment (start 120.65 113.605) (end 120.65 113.03) (width 0.25) (layer B.Cu) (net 13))
 (segment (start 142.87359 142.24) (end 120.65 120.01641) (width 0.25) (layer B.Cu) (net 13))
 (segment (start 151.15 142.24) (end 142.87359 142.24) (width 0.25) (layer B.Cu) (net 13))
 (segment (start 187.96 107.95) (end 187.96 102.87) (width 0.25) (layer B.Cu) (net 14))
 (segment (start 186.69 109.22) (end 187.96 107.95) (width 0.25) (layer B.Cu) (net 14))
 (segment (start 186.69 113.03) (end 186.69 109.22) (width 0.25) (layer B.Cu) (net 14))
 (segment (start 157.48 142.24) (end 152.4 142.24) (width 0.25) (layer B.Cu) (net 14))
 (segment (start 186.69 113.03) (end 157.48 142.24) (width 0.25) (layer B.Cu) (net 14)))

